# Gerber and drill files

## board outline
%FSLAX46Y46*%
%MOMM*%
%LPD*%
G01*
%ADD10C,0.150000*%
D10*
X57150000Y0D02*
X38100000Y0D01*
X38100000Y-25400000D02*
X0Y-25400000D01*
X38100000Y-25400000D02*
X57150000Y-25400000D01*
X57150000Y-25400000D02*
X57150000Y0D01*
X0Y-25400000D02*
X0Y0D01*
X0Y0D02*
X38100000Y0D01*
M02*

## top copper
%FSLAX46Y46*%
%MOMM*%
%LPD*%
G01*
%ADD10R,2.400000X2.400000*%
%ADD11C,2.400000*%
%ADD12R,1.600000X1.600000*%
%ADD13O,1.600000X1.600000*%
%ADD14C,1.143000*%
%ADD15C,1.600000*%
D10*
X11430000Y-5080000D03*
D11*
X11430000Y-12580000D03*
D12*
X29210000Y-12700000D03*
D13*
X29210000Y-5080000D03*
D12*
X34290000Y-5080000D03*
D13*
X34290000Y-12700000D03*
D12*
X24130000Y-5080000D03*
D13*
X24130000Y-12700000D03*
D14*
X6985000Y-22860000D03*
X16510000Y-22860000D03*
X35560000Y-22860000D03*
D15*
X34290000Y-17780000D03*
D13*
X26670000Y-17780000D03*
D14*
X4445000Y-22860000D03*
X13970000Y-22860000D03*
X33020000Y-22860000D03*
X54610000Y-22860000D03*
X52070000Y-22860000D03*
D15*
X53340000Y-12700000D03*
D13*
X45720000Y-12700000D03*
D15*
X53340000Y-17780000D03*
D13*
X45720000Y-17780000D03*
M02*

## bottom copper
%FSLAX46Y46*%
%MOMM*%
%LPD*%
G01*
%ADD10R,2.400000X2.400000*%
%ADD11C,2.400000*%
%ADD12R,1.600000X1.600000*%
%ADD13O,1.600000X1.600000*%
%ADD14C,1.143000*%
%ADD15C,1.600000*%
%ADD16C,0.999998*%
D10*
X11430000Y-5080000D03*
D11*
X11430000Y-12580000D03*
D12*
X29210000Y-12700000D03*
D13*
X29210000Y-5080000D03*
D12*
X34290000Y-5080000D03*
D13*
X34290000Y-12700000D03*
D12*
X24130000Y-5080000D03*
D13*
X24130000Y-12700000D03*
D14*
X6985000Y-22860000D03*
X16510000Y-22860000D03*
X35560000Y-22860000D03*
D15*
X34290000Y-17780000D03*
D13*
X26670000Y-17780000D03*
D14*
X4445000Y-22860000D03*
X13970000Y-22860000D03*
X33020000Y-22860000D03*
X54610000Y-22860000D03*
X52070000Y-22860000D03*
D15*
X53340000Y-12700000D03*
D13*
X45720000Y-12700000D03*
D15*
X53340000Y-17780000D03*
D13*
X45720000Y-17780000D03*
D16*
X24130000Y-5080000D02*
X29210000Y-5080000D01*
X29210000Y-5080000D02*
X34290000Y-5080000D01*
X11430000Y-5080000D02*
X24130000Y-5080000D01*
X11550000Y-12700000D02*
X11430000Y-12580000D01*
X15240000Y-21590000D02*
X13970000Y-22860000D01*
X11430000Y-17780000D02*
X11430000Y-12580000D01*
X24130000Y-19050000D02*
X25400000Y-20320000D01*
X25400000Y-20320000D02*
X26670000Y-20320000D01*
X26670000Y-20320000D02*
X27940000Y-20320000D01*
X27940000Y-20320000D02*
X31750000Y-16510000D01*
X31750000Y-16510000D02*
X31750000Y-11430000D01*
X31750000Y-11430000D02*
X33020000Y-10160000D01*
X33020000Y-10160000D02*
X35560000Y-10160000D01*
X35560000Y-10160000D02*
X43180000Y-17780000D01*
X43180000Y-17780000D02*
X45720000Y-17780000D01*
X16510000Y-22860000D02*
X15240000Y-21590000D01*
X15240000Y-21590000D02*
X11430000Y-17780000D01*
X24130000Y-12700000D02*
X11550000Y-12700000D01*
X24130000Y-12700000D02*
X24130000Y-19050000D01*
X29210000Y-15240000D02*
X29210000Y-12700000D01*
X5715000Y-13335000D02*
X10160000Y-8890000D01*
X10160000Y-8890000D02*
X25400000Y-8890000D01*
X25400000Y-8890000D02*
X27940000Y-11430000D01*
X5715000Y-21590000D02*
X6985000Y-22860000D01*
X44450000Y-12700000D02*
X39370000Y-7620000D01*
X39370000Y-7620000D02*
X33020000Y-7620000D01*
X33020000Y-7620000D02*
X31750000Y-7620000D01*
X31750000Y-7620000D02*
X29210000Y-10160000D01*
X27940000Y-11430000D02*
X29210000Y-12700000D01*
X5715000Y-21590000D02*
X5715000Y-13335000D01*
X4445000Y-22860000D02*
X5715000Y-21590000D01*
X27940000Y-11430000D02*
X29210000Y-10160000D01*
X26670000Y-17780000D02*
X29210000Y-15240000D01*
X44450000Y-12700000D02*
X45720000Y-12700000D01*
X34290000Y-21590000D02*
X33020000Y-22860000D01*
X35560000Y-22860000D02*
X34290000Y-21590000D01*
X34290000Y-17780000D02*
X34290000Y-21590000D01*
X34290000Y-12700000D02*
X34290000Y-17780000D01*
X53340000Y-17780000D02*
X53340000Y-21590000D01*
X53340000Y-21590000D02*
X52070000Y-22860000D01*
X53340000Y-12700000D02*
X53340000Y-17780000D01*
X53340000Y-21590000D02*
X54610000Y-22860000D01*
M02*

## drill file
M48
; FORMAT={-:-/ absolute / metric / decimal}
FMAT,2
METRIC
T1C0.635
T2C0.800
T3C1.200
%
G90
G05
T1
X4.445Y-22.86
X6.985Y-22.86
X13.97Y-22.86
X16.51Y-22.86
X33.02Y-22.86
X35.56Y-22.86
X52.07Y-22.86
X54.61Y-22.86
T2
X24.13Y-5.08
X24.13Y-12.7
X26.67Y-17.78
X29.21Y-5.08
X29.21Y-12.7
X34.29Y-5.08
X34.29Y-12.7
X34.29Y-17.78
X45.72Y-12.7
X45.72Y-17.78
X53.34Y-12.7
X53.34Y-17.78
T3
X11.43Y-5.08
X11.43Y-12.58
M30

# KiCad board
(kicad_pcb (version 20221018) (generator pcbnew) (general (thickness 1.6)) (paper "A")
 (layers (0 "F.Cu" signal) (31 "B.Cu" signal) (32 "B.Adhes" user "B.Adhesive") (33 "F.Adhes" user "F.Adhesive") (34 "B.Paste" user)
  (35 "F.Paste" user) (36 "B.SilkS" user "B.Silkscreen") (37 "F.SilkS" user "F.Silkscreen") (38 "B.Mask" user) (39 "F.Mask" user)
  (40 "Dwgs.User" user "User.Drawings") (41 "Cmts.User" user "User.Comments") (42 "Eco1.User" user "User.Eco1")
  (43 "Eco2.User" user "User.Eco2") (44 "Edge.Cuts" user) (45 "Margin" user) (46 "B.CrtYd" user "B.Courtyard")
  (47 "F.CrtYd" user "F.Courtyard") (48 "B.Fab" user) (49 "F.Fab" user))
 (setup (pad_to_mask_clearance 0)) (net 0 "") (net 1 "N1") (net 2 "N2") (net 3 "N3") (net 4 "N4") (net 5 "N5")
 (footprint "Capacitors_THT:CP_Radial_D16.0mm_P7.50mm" (layer "F.Cu") (at 11.43 5.08 -90)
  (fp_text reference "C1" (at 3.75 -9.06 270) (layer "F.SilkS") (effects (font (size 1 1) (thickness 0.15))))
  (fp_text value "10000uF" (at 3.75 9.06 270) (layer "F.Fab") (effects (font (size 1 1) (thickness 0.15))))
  (pad "1" thru_hole rect (at 0 0 270) (size 2.4 2.4) (drill 1.2) (layers "*.Cu" "*.Mask") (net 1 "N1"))
  (pad "2" thru_hole circle (at 7.5 0 270) (size 2.4 2.4) (drill 1.2) (layers "*.Cu" "*.Mask") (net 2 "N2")))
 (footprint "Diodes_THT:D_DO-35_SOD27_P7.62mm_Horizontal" (layer "F.Cu") (at 29.21 12.7 90)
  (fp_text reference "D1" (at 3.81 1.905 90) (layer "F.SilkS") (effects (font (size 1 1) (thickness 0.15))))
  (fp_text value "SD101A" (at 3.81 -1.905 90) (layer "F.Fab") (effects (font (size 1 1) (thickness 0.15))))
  (pad "1" thru_hole rect (at 0 0 90) (size 1.6 1.6) (drill 0.8) (layers "*.Cu" "*.Mask") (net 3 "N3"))
  (pad "2" thru_hole oval (at 7.62 0 90) (size 1.6 1.6) (drill 0.8) (layers "*.Cu" "*.Mask") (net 1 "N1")))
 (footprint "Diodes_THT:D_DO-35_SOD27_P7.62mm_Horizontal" (layer "F.Cu") (at 34.29 5.08 -90)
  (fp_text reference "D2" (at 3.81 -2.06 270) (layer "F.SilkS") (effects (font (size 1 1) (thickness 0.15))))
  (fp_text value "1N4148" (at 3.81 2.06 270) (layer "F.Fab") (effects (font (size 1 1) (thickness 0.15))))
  (pad "1" thru_hole rect (at 0 0 270) (size 1.6 1.6) (drill 0.8) (layers "*.Cu" "*.Mask") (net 1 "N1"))
  (pad "2" thru_hole oval (at 7.62 0 270) (size 1.6 1.6) (drill 0.8) (layers "*.Cu" "*.Mask") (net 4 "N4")))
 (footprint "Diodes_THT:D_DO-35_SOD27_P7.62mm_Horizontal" (layer "F.Cu") (at 24.13 5.08 -90)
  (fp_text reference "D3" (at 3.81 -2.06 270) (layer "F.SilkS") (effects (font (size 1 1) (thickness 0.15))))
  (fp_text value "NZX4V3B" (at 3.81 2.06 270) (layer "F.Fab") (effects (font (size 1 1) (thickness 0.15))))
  (pad "1" thru_hole rect (at 0 0 270) (size 1.6 1.6) (drill 0.8) (layers "*.Cu" "*.Mask") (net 1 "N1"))
  (pad "2" thru_hole oval (at 7.62 0 270) (size 1.6 1.6) (drill 0.8) (layers "*.Cu" "*.Mask") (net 2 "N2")))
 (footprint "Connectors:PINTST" (layer "F.Cu") (at 6.985 22.86)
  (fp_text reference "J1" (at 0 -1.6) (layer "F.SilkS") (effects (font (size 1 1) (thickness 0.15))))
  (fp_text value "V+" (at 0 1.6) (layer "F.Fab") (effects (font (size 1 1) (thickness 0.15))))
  (pad "1" thru_hole circle (at 0 0) (size 1.143 1.143) (drill 0.635) (layers "*.Cu" "*.Mask") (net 3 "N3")))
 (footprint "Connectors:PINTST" (layer "F.Cu") (at 16.51 22.86)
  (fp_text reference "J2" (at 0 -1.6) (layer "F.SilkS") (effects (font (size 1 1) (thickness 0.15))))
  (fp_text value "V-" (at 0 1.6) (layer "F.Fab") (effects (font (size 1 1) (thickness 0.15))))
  (pad "1" thru_hole circle (at 0 0) (size 1.143 1.143) (drill 0.635) (layers "*.Cu" "*.Mask") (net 2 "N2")))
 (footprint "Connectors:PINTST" (layer "F.Cu") (at 35.56 22.86)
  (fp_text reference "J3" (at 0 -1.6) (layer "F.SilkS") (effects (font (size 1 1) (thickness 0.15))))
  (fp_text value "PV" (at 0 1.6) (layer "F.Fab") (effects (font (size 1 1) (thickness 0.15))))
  (pad "1" thru_hole circle (at 0 0) (size 1.143 1.143) (drill 0.635) (layers "*.Cu" "*.Mask") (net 4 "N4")))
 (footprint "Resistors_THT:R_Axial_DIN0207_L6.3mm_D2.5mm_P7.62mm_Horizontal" (layer "F.Cu") (at 34.29 17.78 180)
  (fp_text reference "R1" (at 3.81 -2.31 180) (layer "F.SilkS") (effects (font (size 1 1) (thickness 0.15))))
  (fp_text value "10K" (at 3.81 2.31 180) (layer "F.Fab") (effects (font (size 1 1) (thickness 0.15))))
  (pad "1" thru_hole circle (at 0 0 180) (size 1.6 1.6) (drill 0.8) (layers "*.Cu" "*.Mask") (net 4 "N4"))
  (pad "2" thru_hole oval (at 7.62 0 180) (size 1.6 1.6) (drill 0.8) (layers "*.Cu" "*.Mask") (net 3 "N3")))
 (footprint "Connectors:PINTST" (layer "F.Cu") (at 4.445 22.86)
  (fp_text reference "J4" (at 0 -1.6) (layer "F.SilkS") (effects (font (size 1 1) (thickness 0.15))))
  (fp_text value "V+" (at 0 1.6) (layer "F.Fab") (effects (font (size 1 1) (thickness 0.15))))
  (pad "1" thru_hole circle (at 0 0) (size 1.143 1.143) (drill 0.635) (layers "*.Cu" "*.Mask") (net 3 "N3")))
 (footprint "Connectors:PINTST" (layer "F.Cu") (at 13.97 22.86)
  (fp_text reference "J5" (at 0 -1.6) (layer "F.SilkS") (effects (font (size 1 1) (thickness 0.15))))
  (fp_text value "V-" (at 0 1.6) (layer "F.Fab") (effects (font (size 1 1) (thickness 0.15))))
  (pad "1" thru_hole circle (at 0 0) (size 1.143 1.143) (drill 0.635) (layers "*.Cu" "*.Mask") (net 2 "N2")))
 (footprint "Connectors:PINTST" (layer "F.Cu") (at 33.02 22.86)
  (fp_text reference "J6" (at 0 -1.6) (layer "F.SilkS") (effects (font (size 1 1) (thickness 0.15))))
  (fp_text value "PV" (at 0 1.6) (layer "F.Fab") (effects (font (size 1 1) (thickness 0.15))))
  (pad "1" thru_hole circle (at 0 0) (size 1.143 1.143) (drill 0.635) (layers "*.Cu" "*.Mask") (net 4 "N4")))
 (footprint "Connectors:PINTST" (layer "F.Cu") (at 54.61 22.86)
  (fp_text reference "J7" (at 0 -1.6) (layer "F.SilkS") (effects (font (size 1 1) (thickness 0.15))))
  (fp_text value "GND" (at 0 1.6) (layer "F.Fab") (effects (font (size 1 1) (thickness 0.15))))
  (pad "1" thru_hole circle (at 0 0) (size 1.143 1.143) (drill 0.635) (layers "*.Cu" "*.Mask") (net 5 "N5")))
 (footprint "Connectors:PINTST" (layer "F.Cu") (at 52.07 22.86)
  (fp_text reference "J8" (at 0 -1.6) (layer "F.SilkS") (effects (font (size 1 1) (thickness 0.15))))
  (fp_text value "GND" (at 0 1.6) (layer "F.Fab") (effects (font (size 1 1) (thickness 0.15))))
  (pad "1" thru_hole circle (at 0 0) (size 1.143 1.143) (drill 0.635) (layers "*.Cu" "*.Mask") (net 5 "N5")))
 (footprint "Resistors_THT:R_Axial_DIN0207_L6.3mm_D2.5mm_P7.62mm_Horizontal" (layer "F.Cu") (at 53.34 12.7 180)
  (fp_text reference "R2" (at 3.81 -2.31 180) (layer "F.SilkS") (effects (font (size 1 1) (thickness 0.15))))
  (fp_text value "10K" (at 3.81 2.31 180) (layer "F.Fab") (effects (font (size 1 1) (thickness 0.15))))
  (pad "1" thru_hole circle (at 0 0 180) (size 1.6 1.6) (drill 0.8) (layers "*.Cu" "*.Mask") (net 5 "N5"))
  (pad "2" thru_hole oval (at 7.62 0 180) (size 1.6 1.6) (drill 0.8) (layers "*.Cu" "*.Mask") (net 3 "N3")))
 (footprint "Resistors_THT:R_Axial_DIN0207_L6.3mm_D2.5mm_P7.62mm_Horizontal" (layer "F.Cu") (at 53.34 17.78 180)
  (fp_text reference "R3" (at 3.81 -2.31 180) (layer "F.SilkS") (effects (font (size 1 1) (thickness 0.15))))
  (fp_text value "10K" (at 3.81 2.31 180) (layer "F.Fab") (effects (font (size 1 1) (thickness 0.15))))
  (pad "1" thru_hole circle (at 0 0 180) (size 1.6 1.6) (drill 0.8) (layers "*.Cu" "*.Mask") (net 5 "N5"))
  (pad "2" thru_hole oval (at 7.62 0 180) (size 1.6 1.6) (drill 0.8) (layers "*.Cu" "*.Mask") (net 2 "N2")))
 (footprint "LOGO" (layer "F.Cu") (at 50.8 6.35)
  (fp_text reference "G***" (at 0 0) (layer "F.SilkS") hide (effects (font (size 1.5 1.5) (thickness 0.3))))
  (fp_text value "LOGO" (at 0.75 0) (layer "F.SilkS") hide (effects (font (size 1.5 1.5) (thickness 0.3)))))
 (gr_line (start 57.15 0) (end 38.1 0) (stroke (width 0.15) (type solid)) (layer "Edge.Cuts"))
 (gr_line (start 38.1 25.4) (end 0 25.4) (stroke (width 0.15) (type solid)) (layer "Edge.Cuts"))
 (gr_line (start 38.1 25.4) (end 57.15 25.4) (stroke (width 0.15) (type solid)) (layer "Edge.Cuts"))
 (gr_line (start 57.15 25.4) (end 57.15 0) (stroke (width 0.15) (type solid)) (layer "Edge.Cuts"))
 (gr_line (start 0 25.4) (end 0 0) (stroke (width 0.15) (type solid)) (layer "Edge.Cuts"))
 (gr_line (start 0 0) (end 38.1 0) (stroke (width 0.15) (type solid)) (layer "Edge.Cuts"))
 (segment (start 24.13 5.08) (end 29.21 5.08) (width 0.999998) (layer "B.Cu") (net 1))
 (segment (start 29.21 5.08) (end 34.29 5.08) (width 0.999998) (layer "B.Cu") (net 1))
 (segment (start 11.43 5.08) (end 24.13 5.08) (width 0.999998) (layer "B.Cu") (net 1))
 (segment (start 11.55 12.7) (end 11.43 12.58) (width 0.999998) (layer "B.Cu") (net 2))
 (segment (start 15.24 21.59) (end 13.97 22.86) (width 0.999998) (layer "B.Cu") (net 2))
 (segment (start 11.43 17.78) (end 11.43 12.58) (width 0.999998) (layer "B.Cu") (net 2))
 (segment (start 24.13 19.05) (end 25.4 20.32) (width 0.999998) (layer "B.Cu") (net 2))
 (segment (start 25.4 20.32) (end 26.67 20.32) (width 0.999998) (layer "B.Cu") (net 2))
 (segment (start 26.67 20.32) (end 27.94 20.32) (width 0.999998) (layer "B.Cu") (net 2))
 (segment (start 27.94 20.32) (end 31.75 16.51) (width 0.999998) (layer "B.Cu") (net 2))
 (segment (start 31.75 16.51) (end 31.75 11.43) (width 0.999998) (layer "B.Cu") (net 2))
 (segment (start 31.75 11.43) (end 33.02 10.16) (width 0.999998) (layer "B.Cu") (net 2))
 (segment (start 33.02 10.16) (end 35.56 10.16) (width 0.999998) (layer "B.Cu") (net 2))
 (segment (start 35.56 10.16) (end 43.18 17.78) (width 0.999998) (layer "B.Cu") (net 2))
 (segment (start 43.18 17.78) (end 45.72 17.78) (width 0.999998) (layer "B.Cu") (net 2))
 (segment (start 16.51 22.86) (end 15.24 21.59) (width 0.999998) (layer "B.Cu") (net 2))
 (segment (start 15.24 21.59) (end 11.43 17.78) (width 0.999998) (layer "B.Cu") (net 2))
 (segment (start 24.13 12.7) (end 11.55 12.7) (width 0.999998) (layer "B.Cu") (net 2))
 (segment (start 24.13 12.7) (end 24.13 19.05) (width 0.999998) (layer "B.Cu") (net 2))
 (segment (start 29.21 15.24) (end 29.21 12.7) (width 0.999998) (layer "B.Cu") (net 3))
 (segment (start 5.715 13.335) (end 10.16 8.89) (width 0.999998) (layer "B.Cu") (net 3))
 (segment (start 10.16 8.89) (end 25.4 8.89) (width 0.999998) (layer "B.Cu") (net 3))
 (segment (start 25.4 8.89) (end 27.94 11.43) (width 0.999998) (layer "B.Cu") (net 3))
 (segment (start 5.715 21.59) (end 6.985 22.86) (width 0.999998) (layer "B.Cu") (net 3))
 (segment (start 44.45 12.7) (end 39.37 7.62) (width 0.999998) (layer "B.Cu") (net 3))
 (segment (start 39.37 7.62) (end 33.02 7.62) (width 0.999998) (layer "B.Cu") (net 3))
 (segment (start 33.02 7.62) (end 31.75 7.62) (width 0.999998) (layer "B.Cu") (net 3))
 (segment (start 31.75 7.62) (end 29.21 10.16) (width 0.999998) (layer "B.Cu") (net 3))
 (segment (start 27.94 11.43) (end 29.21 12.7) (width 0.999998) (layer "B.Cu") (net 3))
 (segment (start 5.715 21.59) (end 5.715 13.335) (width 0.999998) (layer "B.Cu") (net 3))
 (segment (start 4.445 22.86) (end 5.715 21.59) (width 0.999998) (layer "B.Cu") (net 3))
 (segment (start 27.94 11.43) (end 29.21 10.16) (width 0.999998) (layer "B.Cu") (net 3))
 (segment (start 26.67 17.78) (end 29.21 15.24) (width 0.999998) (layer "B.Cu") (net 3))
 (segment (start 44.45 12.7) (end 45.72 12.7) (width 0.999998) (layer "B.Cu") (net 3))
 (segment (start 34.29 21.59) (end 33.02 22.86) (width 0.999998) (layer "B.Cu") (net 4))
 (segment (start 35.56 22.86) (end 34.29 21.59) (width 0.999998) (layer "B.Cu") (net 4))
 (segment (start 34.29 17.78) (end 34.29 21.59) (width 0.999998) (layer "B.Cu") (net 4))
 (segment (start 34.29 12.7) (end 34.29 17.78) (width 0.999998) (layer "B.Cu") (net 4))
 (segment (start 53.34 17.78) (end 53.34 21.59) (width 0.999998) (layer "B.Cu") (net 5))
 (segment (start 53.34 21.59) (end 52.07 22.86) (width 0.999998) (layer "B.Cu") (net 5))
 (segment (start 53.34 12.7) (end 53.34 17.78) (width 0.999998) (layer "B.Cu") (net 5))
 (segment (start 53.34 21.59) (end 54.61 22.86) (width 0.999998) (layer "B.Cu") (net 5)))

